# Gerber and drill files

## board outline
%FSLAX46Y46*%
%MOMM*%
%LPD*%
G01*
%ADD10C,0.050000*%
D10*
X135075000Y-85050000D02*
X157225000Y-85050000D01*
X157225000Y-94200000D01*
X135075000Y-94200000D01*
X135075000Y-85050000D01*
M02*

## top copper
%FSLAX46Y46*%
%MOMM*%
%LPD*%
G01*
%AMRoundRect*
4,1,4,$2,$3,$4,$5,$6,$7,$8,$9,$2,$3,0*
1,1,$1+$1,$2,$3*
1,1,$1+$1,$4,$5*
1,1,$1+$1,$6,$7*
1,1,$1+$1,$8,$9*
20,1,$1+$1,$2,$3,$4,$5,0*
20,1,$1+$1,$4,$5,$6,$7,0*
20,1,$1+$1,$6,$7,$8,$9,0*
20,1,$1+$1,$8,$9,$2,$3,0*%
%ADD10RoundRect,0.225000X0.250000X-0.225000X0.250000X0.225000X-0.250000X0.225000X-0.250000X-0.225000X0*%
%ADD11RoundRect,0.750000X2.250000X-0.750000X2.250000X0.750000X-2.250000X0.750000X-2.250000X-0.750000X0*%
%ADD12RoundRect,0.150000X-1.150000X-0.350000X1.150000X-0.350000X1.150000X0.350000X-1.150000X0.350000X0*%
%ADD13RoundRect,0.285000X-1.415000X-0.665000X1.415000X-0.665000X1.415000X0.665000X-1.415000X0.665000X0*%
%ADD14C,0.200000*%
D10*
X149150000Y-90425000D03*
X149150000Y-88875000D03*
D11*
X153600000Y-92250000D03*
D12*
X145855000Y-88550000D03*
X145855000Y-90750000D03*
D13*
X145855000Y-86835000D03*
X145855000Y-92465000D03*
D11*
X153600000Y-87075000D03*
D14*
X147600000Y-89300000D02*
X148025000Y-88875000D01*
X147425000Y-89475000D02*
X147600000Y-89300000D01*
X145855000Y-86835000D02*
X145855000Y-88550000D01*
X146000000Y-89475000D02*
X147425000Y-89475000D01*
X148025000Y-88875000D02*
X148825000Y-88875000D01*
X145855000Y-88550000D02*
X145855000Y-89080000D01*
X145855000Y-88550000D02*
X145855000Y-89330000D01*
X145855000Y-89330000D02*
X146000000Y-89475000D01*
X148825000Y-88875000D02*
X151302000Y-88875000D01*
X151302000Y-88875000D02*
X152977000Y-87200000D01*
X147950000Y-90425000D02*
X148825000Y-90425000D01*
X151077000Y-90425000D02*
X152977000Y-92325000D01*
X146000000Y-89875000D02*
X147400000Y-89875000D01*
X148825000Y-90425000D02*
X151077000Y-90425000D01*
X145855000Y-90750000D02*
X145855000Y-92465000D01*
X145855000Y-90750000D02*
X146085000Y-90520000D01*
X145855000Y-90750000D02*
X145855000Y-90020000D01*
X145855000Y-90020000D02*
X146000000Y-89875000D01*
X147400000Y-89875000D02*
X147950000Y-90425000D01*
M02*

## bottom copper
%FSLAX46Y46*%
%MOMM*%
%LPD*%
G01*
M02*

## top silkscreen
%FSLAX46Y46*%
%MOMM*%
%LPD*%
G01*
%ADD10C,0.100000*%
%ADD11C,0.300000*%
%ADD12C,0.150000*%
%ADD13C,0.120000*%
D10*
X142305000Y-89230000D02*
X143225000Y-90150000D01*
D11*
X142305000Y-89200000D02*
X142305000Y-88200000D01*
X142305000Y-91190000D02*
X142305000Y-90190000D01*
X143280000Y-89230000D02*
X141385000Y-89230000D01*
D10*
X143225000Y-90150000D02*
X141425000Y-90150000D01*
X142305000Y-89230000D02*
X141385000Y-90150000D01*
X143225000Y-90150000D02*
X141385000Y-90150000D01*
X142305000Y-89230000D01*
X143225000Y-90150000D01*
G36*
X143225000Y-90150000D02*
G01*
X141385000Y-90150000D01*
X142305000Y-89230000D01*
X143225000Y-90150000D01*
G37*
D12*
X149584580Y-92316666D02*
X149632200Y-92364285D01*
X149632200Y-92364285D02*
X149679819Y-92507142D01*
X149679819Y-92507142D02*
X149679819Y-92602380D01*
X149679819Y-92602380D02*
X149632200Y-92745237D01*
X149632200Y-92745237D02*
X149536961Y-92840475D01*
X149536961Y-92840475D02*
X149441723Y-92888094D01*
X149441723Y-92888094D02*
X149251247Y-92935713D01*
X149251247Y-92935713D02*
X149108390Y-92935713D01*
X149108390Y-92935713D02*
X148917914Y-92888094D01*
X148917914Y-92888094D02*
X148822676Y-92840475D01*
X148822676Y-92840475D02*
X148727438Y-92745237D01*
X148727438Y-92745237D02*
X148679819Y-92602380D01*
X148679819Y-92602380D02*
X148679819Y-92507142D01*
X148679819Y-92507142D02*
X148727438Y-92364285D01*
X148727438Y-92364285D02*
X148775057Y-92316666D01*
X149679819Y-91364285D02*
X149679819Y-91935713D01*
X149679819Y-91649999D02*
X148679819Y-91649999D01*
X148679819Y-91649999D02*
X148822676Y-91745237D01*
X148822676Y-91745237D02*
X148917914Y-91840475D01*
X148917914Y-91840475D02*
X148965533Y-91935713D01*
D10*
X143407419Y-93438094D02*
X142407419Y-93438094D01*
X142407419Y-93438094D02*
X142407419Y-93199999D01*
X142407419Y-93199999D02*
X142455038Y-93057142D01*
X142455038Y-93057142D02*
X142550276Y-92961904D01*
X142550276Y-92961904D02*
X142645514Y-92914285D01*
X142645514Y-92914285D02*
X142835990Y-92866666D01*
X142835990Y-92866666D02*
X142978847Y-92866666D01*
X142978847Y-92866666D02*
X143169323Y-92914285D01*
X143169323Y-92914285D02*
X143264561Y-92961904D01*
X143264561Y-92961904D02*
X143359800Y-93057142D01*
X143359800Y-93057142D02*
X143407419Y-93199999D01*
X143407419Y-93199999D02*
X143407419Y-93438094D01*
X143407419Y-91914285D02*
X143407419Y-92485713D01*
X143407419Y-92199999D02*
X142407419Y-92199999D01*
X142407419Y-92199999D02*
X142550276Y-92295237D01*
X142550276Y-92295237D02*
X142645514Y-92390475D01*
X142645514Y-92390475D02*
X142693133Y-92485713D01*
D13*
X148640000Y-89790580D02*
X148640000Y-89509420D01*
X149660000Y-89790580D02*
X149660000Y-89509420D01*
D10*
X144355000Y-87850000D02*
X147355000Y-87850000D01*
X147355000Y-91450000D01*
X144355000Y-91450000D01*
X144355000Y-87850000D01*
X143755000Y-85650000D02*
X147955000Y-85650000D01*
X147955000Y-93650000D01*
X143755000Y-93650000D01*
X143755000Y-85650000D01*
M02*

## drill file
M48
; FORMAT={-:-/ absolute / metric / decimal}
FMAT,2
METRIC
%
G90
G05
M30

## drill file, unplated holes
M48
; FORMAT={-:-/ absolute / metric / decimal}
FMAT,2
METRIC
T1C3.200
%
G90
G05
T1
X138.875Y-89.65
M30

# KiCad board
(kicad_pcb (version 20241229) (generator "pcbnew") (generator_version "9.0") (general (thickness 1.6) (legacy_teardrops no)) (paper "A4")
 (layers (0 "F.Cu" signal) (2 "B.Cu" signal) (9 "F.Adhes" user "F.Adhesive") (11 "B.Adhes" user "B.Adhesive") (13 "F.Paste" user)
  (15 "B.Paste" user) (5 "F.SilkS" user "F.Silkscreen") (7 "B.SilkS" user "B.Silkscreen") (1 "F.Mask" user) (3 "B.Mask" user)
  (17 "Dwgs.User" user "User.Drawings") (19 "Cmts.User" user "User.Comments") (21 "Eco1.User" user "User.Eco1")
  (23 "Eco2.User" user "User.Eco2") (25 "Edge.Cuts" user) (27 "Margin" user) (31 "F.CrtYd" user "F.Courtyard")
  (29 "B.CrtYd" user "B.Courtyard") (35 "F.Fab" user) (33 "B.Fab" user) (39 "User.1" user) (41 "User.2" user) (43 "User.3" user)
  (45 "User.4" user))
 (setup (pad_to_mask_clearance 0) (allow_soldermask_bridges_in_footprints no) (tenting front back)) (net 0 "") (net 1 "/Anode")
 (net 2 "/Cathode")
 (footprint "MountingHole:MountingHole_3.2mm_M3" (layer "F.Cu") (at 138.875 89.65)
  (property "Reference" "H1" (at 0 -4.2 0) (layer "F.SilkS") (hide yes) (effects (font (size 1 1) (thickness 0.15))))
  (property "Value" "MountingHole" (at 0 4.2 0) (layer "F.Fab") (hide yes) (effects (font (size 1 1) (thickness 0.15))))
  (pad "" np_thru_hole circle (at 0 0) (size 3.2 3.2) (drill 3.2) (layers "*.Cu" "*.Mask")))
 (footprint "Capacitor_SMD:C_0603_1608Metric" (layer "F.Cu") (at 149.15 89.65 90)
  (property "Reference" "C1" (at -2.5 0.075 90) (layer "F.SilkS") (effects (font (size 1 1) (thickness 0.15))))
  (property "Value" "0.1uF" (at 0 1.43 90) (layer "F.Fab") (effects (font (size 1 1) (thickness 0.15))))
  (fp_line (start -0.14058 -0.51) (end 0.14058 -0.51) (stroke (width 0.12) (type solid)) (layer "F.SilkS"))
  (fp_line (start -0.14058 0.51) (end 0.14058 0.51) (stroke (width 0.12) (type solid)) (layer "F.SilkS"))
  (pad "1" smd roundrect (at -0.775 0 90) (size 0.9 0.95) (layers "F.Cu" "F.Mask" "F.Paste") (roundrect_rratio 0.25) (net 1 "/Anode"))
  (pad "2" smd roundrect (at 0.775 0 90) (size 0.9 0.95) (layers "F.Cu" "F.Mask" "F.Paste") (roundrect_rratio 0.25) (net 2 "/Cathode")))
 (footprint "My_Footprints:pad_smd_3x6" (layer "F.Cu") (at 153.6 92.25)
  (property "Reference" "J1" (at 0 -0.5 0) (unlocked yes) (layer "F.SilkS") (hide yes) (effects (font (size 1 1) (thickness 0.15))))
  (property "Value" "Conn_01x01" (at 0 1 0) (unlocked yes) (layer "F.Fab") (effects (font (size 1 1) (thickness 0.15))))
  (pad "1" smd roundrect (at 0 0 90) (size 3 6) (layers "F.Cu" "F.Mask" "F.Paste") (roundrect_rratio 0.25) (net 1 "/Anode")
   (thermal_bridge_angle 45)))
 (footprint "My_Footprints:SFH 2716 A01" (layer "F.Cu") (at 145.855 89.65)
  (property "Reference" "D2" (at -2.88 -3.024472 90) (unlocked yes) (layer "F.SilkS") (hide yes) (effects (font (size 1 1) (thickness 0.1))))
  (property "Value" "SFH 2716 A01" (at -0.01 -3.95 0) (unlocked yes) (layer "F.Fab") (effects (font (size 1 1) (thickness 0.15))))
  (fp_rect (start -1.5 -1.8) (end 1.5 1.8) (stroke (width 0.1) (type solid)) (fill no) (layer "F.SilkS"))
  (pad "1" smd roundrect (at 0 -1.1) (size 2.6 1) (layers "F.Cu" "F.Mask" "F.Paste") (roundrect_rratio 0.15) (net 2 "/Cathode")
   (thermal_bridge_angle 45))
  (pad "2" smd roundrect (at 0 1.1) (size 2.6 1) (layers "F.Cu" "F.Mask" "F.Paste") (roundrect_rratio 0.15) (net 1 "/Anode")
   (thermal_bridge_angle 45)))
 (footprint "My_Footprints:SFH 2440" (layer "F.Cu") (at 145.855 89.65)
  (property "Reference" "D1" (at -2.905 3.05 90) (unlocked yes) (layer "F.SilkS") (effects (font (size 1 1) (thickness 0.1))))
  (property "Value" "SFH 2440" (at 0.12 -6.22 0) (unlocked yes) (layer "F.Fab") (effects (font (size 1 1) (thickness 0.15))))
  (fp_rect (start -2.1 -4) (end 2.1 4) (stroke (width 0.1) (type solid)) (fill no) (layer "F.SilkS"))
  (pad "1" smd roundrect (at 0 -2.815) (size 3.4 1.9) (layers "F.Cu" "F.Mask" "F.Paste") (roundrect_rratio 0.15) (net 2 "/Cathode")
   (thermal_bridge_angle 45))
  (pad "2" smd roundrect (at 0 2.815) (size 3.4 1.9) (layers "F.Cu" "F.Mask" "F.Paste") (roundrect_rratio 0.15) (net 1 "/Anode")
   (thermal_bridge_angle 45)))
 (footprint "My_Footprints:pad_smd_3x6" (layer "F.Cu") (at 153.6 87.075)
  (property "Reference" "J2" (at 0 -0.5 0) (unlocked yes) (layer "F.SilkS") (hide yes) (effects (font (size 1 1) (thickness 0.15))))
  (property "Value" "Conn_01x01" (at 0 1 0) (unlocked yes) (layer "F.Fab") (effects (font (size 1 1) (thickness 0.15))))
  (pad "1" smd roundrect (at 0 0 90) (size 3 6) (layers "F.Cu" "F.Mask" "F.Paste") (roundrect_rratio 0.25) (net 2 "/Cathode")
   (thermal_bridge_angle 45)))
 (gr_line (start 142.305 89.23) (end 143.225 90.15) (stroke (width 0.1) (type default)) (layer "F.SilkS"))
 (gr_line (start 142.305 89.2) (end 142.305 88.2) (stroke (width 0.3) (type solid)) (layer "F.SilkS"))
 (gr_line (start 142.305 91.19) (end 142.305 90.19) (stroke (width 0.3) (type solid)) (layer "F.SilkS"))
 (gr_line (start 143.28 89.23) (end 141.385 89.23) (stroke (width 0.3) (type solid)) (layer "F.SilkS"))
 (gr_line (start 143.225 90.15) (end 141.425 90.15) (stroke (width 0.1) (type default)) (layer "F.SilkS"))
 (gr_line (start 142.305 89.23) (end 141.385 90.15) (stroke (width 0.1) (type default)) (layer "F.SilkS"))
 (gr_poly (pts (xy 141.385 90.15) (xy 142.305 89.23) (xy 143.225 90.15)) (stroke (width 0.1) (type solid)) (fill yes) (layer "F.SilkS"))
 (gr_rect (start 135.075 85.05) (end 157.225 94.2) (stroke (width 0.05) (type default)) (fill no) (layer "Edge.Cuts"))
 (segment (start 147.6 89.3) (end 148.025 88.875) (width 0.2) (layer "F.Cu") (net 2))
 (segment (start 147.425 89.475) (end 147.6 89.3) (width 0.2) (layer "F.Cu") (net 2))
 (segment (start 145.855 86.835) (end 145.855 88.55) (width 0.2) (layer "F.Cu") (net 2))
 (segment (start 146 89.475) (end 147.425 89.475) (width 0.2) (layer "F.Cu") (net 2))
 (segment (start 148.025 88.875) (end 148.825 88.875) (width 0.2) (layer "F.Cu") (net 2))
 (segment (start 145.855 88.55) (end 145.855 89.08) (width 0.2) (layer "F.Cu") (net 2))
 (segment (start 145.855 88.55) (end 145.855 89.33) (width 0.2) (layer "F.Cu") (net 2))
 (segment (start 145.855 89.33) (end 146 89.475) (width 0.2) (layer "F.Cu") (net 2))
 (segment (start 148.825 88.875) (end 151.302 88.875) (width 0.2) (layer "F.Cu") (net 2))
 (segment (start 151.302 88.875) (end 152.977 87.2) (width 0.2) (layer "F.Cu") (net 2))
 (segment (start 147.95 90.425) (end 148.825 90.425) (width 0.2) (layer "F.Cu") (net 1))
 (segment (start 151.077 90.425) (end 152.977 92.325) (width 0.2) (layer "F.Cu") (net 1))
 (segment (start 146 89.875) (end 147.4 89.875) (width 0.2) (layer "F.Cu") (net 1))
 (segment (start 148.825 90.425) (end 151.077 90.425) (width 0.2) (layer "F.Cu") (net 1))
 (segment (start 145.855 90.75) (end 145.855 92.465) (width 0.2) (layer "F.Cu") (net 1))
 (segment (start 145.855 90.75) (end 146.085 90.52) (width 0.2) (layer "F.Cu") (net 1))
 (segment (start 145.855 90.75) (end 145.855 90.02) (width 0.2) (layer "F.Cu") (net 1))
 (segment (start 145.855 90.02) (end 146 89.875) (width 0.2) (layer "F.Cu") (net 1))
 (segment (start 147.4 89.875) (end 147.95 90.425) (width 0.2) (layer "F.Cu") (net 1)))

